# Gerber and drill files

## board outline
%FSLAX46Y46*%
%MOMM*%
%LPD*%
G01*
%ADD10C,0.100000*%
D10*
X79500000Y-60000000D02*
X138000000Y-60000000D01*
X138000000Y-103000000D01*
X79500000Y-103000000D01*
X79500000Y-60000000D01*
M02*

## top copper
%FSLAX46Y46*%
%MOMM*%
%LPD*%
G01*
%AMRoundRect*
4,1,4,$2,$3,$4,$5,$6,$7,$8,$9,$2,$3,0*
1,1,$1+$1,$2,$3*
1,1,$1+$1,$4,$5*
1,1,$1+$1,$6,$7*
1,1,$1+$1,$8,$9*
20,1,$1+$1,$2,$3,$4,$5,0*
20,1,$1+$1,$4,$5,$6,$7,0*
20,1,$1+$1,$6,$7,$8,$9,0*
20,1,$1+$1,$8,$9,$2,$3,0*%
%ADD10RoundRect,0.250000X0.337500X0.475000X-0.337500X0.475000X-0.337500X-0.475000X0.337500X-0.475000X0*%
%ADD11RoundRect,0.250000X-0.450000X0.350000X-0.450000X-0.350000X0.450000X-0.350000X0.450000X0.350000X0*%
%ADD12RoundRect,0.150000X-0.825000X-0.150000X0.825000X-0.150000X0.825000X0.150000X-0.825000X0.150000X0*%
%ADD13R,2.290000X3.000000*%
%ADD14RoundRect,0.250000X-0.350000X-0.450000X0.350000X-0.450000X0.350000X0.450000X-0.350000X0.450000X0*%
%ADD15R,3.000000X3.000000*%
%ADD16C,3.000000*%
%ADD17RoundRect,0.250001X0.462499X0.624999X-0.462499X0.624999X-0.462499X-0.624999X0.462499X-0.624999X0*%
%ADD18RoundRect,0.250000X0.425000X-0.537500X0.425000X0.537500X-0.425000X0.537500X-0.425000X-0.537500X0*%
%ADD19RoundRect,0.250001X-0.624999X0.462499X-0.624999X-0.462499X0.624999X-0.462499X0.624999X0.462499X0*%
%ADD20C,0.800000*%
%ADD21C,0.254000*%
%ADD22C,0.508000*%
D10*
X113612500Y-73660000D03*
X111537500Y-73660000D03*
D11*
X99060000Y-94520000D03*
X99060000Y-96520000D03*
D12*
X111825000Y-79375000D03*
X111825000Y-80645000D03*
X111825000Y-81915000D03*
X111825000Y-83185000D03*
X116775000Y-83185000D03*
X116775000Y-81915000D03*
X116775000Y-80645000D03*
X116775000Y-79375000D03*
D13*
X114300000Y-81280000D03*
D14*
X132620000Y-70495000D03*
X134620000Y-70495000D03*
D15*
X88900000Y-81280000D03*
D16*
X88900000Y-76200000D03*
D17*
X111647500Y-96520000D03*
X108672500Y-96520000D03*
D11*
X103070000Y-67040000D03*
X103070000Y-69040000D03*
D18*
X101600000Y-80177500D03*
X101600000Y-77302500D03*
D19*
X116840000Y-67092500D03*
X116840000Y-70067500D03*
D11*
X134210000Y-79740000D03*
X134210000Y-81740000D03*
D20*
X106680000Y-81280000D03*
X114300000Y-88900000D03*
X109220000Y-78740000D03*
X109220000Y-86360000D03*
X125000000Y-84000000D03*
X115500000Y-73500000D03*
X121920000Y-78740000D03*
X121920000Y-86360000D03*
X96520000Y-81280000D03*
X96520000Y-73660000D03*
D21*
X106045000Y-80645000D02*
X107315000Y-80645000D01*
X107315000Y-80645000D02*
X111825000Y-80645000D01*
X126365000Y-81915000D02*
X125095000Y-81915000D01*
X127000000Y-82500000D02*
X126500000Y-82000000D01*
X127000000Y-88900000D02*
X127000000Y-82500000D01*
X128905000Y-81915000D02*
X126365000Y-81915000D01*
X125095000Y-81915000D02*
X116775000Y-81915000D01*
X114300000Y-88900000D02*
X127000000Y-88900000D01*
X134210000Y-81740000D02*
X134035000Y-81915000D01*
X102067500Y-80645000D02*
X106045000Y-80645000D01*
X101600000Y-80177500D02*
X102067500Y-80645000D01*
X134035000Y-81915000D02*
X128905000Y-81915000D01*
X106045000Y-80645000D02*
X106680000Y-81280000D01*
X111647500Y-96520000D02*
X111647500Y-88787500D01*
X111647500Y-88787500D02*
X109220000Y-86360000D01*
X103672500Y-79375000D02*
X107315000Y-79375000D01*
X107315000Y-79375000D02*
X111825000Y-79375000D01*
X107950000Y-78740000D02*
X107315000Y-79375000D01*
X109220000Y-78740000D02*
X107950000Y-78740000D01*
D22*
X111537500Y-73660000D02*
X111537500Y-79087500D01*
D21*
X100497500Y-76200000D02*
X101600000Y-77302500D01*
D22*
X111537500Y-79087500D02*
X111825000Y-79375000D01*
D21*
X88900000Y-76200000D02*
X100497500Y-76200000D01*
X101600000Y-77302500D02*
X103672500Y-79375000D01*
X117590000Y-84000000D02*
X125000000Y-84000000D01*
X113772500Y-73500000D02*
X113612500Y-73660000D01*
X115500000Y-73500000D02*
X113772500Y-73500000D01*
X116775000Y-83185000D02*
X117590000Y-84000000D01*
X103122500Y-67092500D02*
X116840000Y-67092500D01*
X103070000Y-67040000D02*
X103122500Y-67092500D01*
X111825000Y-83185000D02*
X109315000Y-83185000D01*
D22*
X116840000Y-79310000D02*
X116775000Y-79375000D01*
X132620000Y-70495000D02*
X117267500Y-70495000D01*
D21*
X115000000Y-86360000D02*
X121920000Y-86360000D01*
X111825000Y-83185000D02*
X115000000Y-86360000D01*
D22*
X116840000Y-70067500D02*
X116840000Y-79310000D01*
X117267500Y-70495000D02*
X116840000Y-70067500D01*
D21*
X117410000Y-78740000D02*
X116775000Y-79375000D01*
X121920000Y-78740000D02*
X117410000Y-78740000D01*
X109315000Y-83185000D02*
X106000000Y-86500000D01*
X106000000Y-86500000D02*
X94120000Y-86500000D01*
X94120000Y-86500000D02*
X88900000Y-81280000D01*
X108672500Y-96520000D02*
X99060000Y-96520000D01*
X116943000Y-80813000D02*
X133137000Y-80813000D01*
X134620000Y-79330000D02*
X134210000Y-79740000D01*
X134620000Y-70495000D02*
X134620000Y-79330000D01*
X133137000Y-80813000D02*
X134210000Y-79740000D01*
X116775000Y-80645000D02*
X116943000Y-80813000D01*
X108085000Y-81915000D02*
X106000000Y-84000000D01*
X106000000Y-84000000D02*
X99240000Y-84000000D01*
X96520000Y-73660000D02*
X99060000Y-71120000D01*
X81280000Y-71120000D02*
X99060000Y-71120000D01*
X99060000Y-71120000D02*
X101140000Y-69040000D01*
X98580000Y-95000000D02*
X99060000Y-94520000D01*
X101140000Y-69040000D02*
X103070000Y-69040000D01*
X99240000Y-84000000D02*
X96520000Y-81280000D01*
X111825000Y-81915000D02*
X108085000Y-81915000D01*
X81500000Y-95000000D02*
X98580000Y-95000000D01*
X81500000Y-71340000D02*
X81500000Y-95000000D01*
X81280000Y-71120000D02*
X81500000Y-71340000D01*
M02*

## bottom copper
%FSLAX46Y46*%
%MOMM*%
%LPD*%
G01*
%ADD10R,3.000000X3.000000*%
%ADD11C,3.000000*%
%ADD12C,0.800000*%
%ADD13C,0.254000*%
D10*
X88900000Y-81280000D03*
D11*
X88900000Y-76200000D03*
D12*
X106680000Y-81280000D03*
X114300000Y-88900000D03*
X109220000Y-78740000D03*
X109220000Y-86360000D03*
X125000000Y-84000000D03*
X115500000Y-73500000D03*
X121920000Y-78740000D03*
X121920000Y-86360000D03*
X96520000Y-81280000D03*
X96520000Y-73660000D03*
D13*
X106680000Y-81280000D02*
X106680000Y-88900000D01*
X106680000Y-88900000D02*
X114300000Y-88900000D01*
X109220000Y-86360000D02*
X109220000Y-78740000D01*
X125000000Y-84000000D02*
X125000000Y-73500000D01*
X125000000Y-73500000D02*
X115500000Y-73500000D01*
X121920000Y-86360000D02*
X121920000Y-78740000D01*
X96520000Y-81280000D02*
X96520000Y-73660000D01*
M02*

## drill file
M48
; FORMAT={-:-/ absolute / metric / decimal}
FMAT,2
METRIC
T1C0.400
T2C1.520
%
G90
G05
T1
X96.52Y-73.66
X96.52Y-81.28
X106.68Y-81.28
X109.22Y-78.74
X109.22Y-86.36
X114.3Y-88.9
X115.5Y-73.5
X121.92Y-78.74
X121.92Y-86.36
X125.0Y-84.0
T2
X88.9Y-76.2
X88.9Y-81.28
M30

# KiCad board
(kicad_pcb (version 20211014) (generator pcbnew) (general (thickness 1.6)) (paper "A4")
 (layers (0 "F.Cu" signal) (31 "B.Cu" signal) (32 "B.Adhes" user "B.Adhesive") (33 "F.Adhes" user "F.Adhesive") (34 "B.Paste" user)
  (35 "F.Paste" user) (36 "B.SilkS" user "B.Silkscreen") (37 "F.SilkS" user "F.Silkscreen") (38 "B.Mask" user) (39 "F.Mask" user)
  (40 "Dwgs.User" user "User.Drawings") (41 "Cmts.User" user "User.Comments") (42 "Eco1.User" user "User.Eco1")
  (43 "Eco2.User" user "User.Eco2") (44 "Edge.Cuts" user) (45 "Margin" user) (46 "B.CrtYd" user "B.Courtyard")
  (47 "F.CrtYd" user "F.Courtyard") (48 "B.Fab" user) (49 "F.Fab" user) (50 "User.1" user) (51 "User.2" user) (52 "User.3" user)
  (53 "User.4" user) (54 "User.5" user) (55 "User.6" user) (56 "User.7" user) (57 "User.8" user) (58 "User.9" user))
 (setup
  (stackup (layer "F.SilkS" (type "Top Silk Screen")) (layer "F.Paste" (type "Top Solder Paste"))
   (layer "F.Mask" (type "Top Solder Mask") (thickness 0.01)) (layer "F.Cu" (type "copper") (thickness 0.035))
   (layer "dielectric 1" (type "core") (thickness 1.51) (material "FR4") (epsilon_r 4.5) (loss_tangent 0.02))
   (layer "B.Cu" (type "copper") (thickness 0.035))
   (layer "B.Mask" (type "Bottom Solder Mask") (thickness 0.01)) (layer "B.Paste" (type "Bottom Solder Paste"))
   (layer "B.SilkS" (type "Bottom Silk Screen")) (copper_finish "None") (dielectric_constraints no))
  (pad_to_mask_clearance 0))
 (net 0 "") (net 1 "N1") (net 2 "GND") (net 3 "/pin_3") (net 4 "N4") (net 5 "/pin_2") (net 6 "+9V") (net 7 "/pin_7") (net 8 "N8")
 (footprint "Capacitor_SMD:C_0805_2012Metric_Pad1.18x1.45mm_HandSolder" (layer "F.Cu") (at 112.575 73.66 180)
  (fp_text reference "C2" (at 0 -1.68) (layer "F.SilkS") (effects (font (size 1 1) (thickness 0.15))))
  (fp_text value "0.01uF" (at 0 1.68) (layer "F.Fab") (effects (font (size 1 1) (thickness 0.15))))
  (pad "1" smd roundrect (at -1.0375 0 180) (size 1.175 1.45) (layers "F.Cu" "F.Paste" "F.Mask") (roundrect_rratio 0.2127659574)
   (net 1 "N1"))
  (pad "2" smd roundrect (at 1.0375 0 180) (size 1.175 1.45) (layers "F.Cu" "F.Paste" "F.Mask") (roundrect_rratio 0.2127659574)
   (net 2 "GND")))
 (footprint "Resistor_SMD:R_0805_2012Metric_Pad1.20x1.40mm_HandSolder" (layer "F.Cu") (at 99.06 95.52 -90)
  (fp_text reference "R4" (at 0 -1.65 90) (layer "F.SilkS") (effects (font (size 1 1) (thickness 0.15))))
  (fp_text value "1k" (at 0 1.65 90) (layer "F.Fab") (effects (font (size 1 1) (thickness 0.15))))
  (pad "1" smd roundrect (at -1 0 270) (size 1.2 1.4) (layers "F.Cu" "F.Paste" "F.Mask") (roundrect_rratio 0.2083333333) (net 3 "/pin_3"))
  (pad "2" smd roundrect (at 1 0 270) (size 1.2 1.4) (layers "F.Cu" "F.Paste" "F.Mask") (roundrect_rratio 0.2083333333) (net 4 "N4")))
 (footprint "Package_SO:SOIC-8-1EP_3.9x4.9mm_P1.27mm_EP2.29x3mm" (layer "F.Cu") (at 114.3 81.28)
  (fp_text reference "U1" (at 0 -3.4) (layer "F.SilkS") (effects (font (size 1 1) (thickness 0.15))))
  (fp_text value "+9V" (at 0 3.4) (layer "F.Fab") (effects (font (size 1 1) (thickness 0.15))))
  (pad "" smd roundrect (at 0.57 0.75) (size 0.92 1.21) (layers "F.Paste") (roundrect_rratio 0.25))
  (pad "" smd roundrect (at 0.57 -0.75) (size 0.92 1.21) (layers "F.Paste") (roundrect_rratio 0.25))
  (pad "" smd roundrect (at -0.57 -0.75) (size 0.92 1.21) (layers "F.Paste") (roundrect_rratio 0.25))
  (pad "" smd roundrect (at -0.57 0.75) (size 0.92 1.21) (layers "F.Paste") (roundrect_rratio 0.25))
  (pad "1" smd roundrect (at -2.475 -1.905) (size 1.95 0.6) (layers "F.Cu" "F.Paste" "F.Mask") (roundrect_rratio 0.25) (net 2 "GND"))
  (pad "2" smd roundrect (at -2.475 -0.635) (size 1.95 0.6) (layers "F.Cu" "F.Paste" "F.Mask") (roundrect_rratio 0.25) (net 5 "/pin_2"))
  (pad "3" smd roundrect (at -2.475 0.635) (size 1.95 0.6) (layers "F.Cu" "F.Paste" "F.Mask") (roundrect_rratio 0.25) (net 3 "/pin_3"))
  (pad "4" smd roundrect (at -2.475 1.905) (size 1.95 0.6) (layers "F.Cu" "F.Paste" "F.Mask") (roundrect_rratio 0.25) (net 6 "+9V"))
  (pad "5" smd roundrect (at 2.475 1.905) (size 1.95 0.6) (layers "F.Cu" "F.Paste" "F.Mask") (roundrect_rratio 0.25) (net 1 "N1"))
  (pad "6" smd roundrect (at 2.475 0.635) (size 1.95 0.6) (layers "F.Cu" "F.Paste" "F.Mask") (roundrect_rratio 0.25) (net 5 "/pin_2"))
  (pad "7" smd roundrect (at 2.475 -0.635) (size 1.95 0.6) (layers "F.Cu" "F.Paste" "F.Mask") (roundrect_rratio 0.25) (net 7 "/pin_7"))
  (pad "8" smd roundrect (at 2.475 -1.905) (size 1.95 0.6) (layers "F.Cu" "F.Paste" "F.Mask") (roundrect_rratio 0.25) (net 6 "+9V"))
  (pad "9" smd rect (at 0 0) (size 2.29 3) (layers "F.Cu" "F.Mask")))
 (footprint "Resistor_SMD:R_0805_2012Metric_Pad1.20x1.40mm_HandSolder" (layer "F.Cu") (at 133.62 70.495)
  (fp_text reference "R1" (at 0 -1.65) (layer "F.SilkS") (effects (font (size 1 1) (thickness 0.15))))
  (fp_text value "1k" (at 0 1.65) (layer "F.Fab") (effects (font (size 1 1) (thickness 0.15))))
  (pad "1" smd roundrect (at -1 0) (size 1.2 1.4) (layers "F.Cu" "F.Paste" "F.Mask") (roundrect_rratio 0.2083333333) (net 6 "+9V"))
  (pad "2" smd roundrect (at 1 0) (size 1.2 1.4) (layers "F.Cu" "F.Paste" "F.Mask") (roundrect_rratio 0.2083333333) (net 7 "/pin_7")))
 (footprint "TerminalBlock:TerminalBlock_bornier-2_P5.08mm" (layer "F.Cu") (at 88.9 81.28 90)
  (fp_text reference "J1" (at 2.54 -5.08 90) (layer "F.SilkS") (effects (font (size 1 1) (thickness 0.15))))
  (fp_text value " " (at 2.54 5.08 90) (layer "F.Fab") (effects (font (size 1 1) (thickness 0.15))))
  (pad "1" thru_hole rect (at 0 0 90) (size 3 3) (drill 1.52) (layers *.Cu *.Mask) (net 6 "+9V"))
  (pad "2" thru_hole circle (at 5.08 0 90) (size 3 3) (drill 1.52) (layers *.Cu *.Mask) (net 2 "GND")))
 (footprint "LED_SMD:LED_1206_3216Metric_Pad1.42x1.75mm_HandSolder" (layer "F.Cu") (at 110.16 96.52 180)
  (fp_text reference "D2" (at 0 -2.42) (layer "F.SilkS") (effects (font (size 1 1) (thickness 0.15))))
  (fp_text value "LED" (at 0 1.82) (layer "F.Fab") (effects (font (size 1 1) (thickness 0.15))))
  (pad "1" smd roundrect (at -1.4875 0 180) (size 1.425 1.75) (layers "F.Cu" "F.Paste" "F.Mask") (roundrect_rratio 0.1754392982)
   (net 2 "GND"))
  (pad "2" smd roundrect (at 1.4875 0 180) (size 1.425 1.75) (layers "F.Cu" "F.Paste" "F.Mask") (roundrect_rratio 0.1754392982) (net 4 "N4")))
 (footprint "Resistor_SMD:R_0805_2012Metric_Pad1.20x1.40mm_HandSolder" (layer "F.Cu") (at 103.07 68.04 -90)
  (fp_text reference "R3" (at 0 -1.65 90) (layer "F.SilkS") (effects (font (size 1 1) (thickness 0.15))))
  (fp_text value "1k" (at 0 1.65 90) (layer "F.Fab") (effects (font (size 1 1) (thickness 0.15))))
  (pad "1" smd roundrect (at -1 0 270) (size 1.2 1.4) (layers "F.Cu" "F.Paste" "F.Mask") (roundrect_rratio 0.2083333333) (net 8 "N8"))
  (pad "2" smd roundrect (at 1 0 270) (size 1.2 1.4) (layers "F.Cu" "F.Paste" "F.Mask") (roundrect_rratio 0.2083333333) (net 3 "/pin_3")))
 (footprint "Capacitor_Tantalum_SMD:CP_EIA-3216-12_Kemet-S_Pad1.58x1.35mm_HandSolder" (layer "F.Cu") (at 101.6 78.74 90)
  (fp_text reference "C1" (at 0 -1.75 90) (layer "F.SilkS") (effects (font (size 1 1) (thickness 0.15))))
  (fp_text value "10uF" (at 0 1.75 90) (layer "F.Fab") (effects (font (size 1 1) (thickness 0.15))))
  (pad "1" smd roundrect (at -1.4375 0 90) (size 1.575 1.35) (layers "F.Cu" "F.Paste" "F.Mask") (roundrect_rratio 0.1851851852)
   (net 5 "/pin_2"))
  (pad "2" smd roundrect (at 1.4375 0 90) (size 1.575 1.35) (layers "F.Cu" "F.Paste" "F.Mask") (roundrect_rratio 0.1851851852) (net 2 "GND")))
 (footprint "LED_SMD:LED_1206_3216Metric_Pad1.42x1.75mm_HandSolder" (layer "F.Cu") (at 116.84 68.58 -90)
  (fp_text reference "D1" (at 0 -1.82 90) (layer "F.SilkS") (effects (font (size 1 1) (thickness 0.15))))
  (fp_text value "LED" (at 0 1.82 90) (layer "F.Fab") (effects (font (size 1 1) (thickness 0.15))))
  (pad "1" smd roundrect (at -1.4875 0 270) (size 1.425 1.75) (layers "F.Cu" "F.Paste" "F.Mask") (roundrect_rratio 0.1754392982)
   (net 8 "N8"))
  (pad "2" smd roundrect (at 1.4875 0 270) (size 1.425 1.75) (layers "F.Cu" "F.Paste" "F.Mask") (roundrect_rratio 0.1754392982)
   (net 6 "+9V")))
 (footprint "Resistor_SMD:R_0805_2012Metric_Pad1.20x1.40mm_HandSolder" (layer "F.Cu") (at 134.21 80.74 -90)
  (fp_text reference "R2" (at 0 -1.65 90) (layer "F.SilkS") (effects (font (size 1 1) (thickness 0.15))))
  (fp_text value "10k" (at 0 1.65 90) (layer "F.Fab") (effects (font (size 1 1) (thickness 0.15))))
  (pad "1" smd roundrect (at -1 0 270) (size 1.2 1.4) (layers "F.Cu" "F.Paste" "F.Mask") (roundrect_rratio 0.2083333333) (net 7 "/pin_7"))
  (pad "2" smd roundrect (at 1 0 270) (size 1.2 1.4) (layers "F.Cu" "F.Paste" "F.Mask") (roundrect_rratio 0.2083333333) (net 5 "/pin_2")))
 (gr_rect (start 79.5 60) (end 138 103) (layer "Edge.Cuts") (width 0.1) (fill none))
 (segment (start 106.045 80.645) (end 107.315 80.645) (width 0.254) (layer "F.Cu") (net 5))
 (segment (start 107.315 80.645) (end 111.825 80.645) (width 0.254) (layer "F.Cu") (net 5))
 (segment (start 126.365 81.915) (end 125.095 81.915) (width 0.254) (layer "F.Cu") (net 5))
 (segment (start 127 82.5) (end 126.5 82) (width 0.254) (layer "F.Cu") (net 5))
 (segment (start 127 88.9) (end 127 82.5) (width 0.254) (layer "F.Cu") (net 5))
 (segment (start 128.905 81.915) (end 126.365 81.915) (width 0.254) (layer "F.Cu") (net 5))
 (segment (start 125.095 81.915) (end 116.775 81.915) (width 0.254) (layer "F.Cu") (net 5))
 (segment (start 114.3 88.9) (end 127 88.9) (width 0.254) (layer "F.Cu") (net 5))
 (segment (start 134.21 81.74) (end 134.035 81.915) (width 0.254) (layer "F.Cu") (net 5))
 (segment (start 102.0675 80.645) (end 106.045 80.645) (width 0.254) (layer "F.Cu") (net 5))
 (segment (start 101.6 80.1775) (end 102.0675 80.645) (width 0.254) (layer "F.Cu") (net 5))
 (segment (start 134.035 81.915) (end 128.905 81.915) (width 0.254) (layer "F.Cu") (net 5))
 (segment (start 106.045 80.645) (end 106.68 81.28) (width 0.254) (layer "F.Cu") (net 5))
 (via (at 106.68 81.28) (size 0.8) (drill 0.4) (layers "F.Cu" "B.Cu") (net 5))
 (via (at 114.3 88.9) (size 0.8) (drill 0.4) (layers "F.Cu" "B.Cu") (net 5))
 (segment (start 106.68 81.28) (end 106.68 88.9) (width 0.254) (layer "B.Cu") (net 5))
 (segment (start 106.68 88.9) (end 114.3 88.9) (width 0.254) (layer "B.Cu") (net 5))
 (segment (start 111.6475 96.52) (end 111.6475 88.7875) (width 0.254) (layer "F.Cu") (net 2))
 (segment (start 111.6475 88.7875) (end 109.22 86.36) (width 0.254) (layer "F.Cu") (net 2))
 (segment (start 103.6725 79.375) (end 107.315 79.375) (width 0.254) (layer "F.Cu") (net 2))
 (segment (start 107.315 79.375) (end 111.825 79.375) (width 0.254) (layer "F.Cu") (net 2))
 (segment (start 107.95 78.74) (end 107.315 79.375) (width 0.254) (layer "F.Cu") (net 2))
 (segment (start 109.22 78.74) (end 107.95 78.74) (width 0.254) (layer "F.Cu") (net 2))
 (segment (start 111.5375 73.66) (end 111.5375 79.0875) (width 0.508) (layer "F.Cu") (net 2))
 (segment (start 100.4975 76.2) (end 101.6 77.3025) (width 0.254) (layer "F.Cu") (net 2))
 (segment (start 111.5375 79.0875) (end 111.825 79.375) (width 0.508) (layer "F.Cu") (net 2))
 (segment (start 88.9 76.2) (end 100.4975 76.2) (width 0.254) (layer "F.Cu") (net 2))
 (segment (start 101.6 77.3025) (end 103.6725 79.375) (width 0.254) (layer "F.Cu") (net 2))
 (via (at 109.22 78.74) (size 0.8) (drill 0.4) (layers "F.Cu" "B.Cu") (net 2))
 (via (at 109.22 86.36) (size 0.8) (drill 0.4) (layers "F.Cu" "B.Cu") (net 2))
 (segment (start 109.22 86.36) (end 109.22 78.74) (width 0.254) (layer "B.Cu") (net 2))
 (segment (start 117.59 84) (end 125 84) (width 0.254) (layer "F.Cu") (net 1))
 (segment (start 113.7725 73.5) (end 113.6125 73.66) (width 0.254) (layer "F.Cu") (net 1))
 (segment (start 115.5 73.5) (end 113.7725 73.5) (width 0.254) (layer "F.Cu") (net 1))
 (segment (start 116.775 83.185) (end 117.59 84) (width 0.254) (layer "F.Cu") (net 1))
 (via (at 125 84) (size 0.8) (drill 0.4) (layers "F.Cu" "B.Cu") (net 1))
 (via (at 115.5 73.5) (size 0.8) (drill 0.4) (layers "F.Cu" "B.Cu") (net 1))
 (segment (start 125 84) (end 125 73.5) (width 0.254) (layer "B.Cu") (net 1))
 (segment (start 125 73.5) (end 115.5 73.5) (width 0.254) (layer "B.Cu") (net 1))
 (segment (start 103.1225 67.0925) (end 116.84 67.0925) (width 0.254) (layer "F.Cu") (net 8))
 (segment (start 103.07 67.04) (end 103.1225 67.0925) (width 0.254) (layer "F.Cu") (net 8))
 (segment (start 111.825 83.185) (end 109.315 83.185) (width 0.254) (layer "F.Cu") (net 6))
 (segment (start 116.84 79.31) (end 116.775 79.375) (width 0.508) (layer "F.Cu") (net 6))
 (segment (start 132.62 70.495) (end 117.2675 70.495) (width 0.508) (layer "F.Cu") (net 6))
 (segment (start 115 86.36) (end 121.92 86.36) (width 0.254) (layer "F.Cu") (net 6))
 (segment (start 111.825 83.185) (end 115 86.36) (width 0.254) (layer "F.Cu") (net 6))
 (segment (start 116.84 70.0675) (end 116.84 79.31) (width 0.508) (layer "F.Cu") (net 6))
 (segment (start 117.2675 70.495) (end 116.84 70.0675) (width 0.508) (layer "F.Cu") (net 6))
 (segment (start 117.41 78.74) (end 116.775 79.375) (width 0.254) (layer "F.Cu") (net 6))
 (segment (start 121.92 78.74) (end 117.41 78.74) (width 0.254) (layer "F.Cu") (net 6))
 (segment (start 109.315 83.185) (end 106 86.5) (width 0.254) (layer "F.Cu") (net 6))
 (segment (start 106 86.5) (end 94.12 86.5) (width 0.254) (layer "F.Cu") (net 6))
 (segment (start 94.12 86.5) (end 88.9 81.28) (width 0.254) (layer "F.Cu") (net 6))
 (via (at 121.92 78.74) (size 0.8) (drill 0.4) (layers "F.Cu" "B.Cu") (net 6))
 (via (at 121.92 86.36) (size 0.8) (drill 0.4) (layers "F.Cu" "B.Cu") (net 6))
 (segment (start 121.92 86.36) (end 121.92 78.74) (width 0.254) (layer "B.Cu") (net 6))
 (segment (start 108.6725 96.52) (end 99.06 96.52) (width 0.254) (layer "F.Cu") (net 4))
 (segment (start 116.943 80.813) (end 133.137 80.813) (width 0.254) (layer "F.Cu") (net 7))
 (segment (start 134.62 79.33) (end 134.21 79.74) (width 0.254) (layer "F.Cu") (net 7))
 (segment (start 134.62 70.495) (end 134.62 79.33) (width 0.254) (layer "F.Cu") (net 7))
 (segment (start 133.137 80.813) (end 134.21 79.74) (width 0.254) (layer "F.Cu") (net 7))
 (segment (start 116.775 80.645) (end 116.943 80.813) (width 0.254) (layer "F.Cu") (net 7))
 (segment (start 108.085 81.915) (end 106 84) (width 0.254) (layer "F.Cu") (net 3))
 (segment (start 106 84) (end 99.24 84) (width 0.254) (layer "F.Cu") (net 3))
 (segment (start 96.52 73.66) (end 99.06 71.12) (width 0.254) (layer "F.Cu") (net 3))
 (segment (start 81.28 71.12) (end 99.06 71.12) (width 0.254) (layer "F.Cu") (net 3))
 (segment (start 99.06 71.12) (end 101.14 69.04) (width 0.254) (layer "F.Cu") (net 3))
 (segment (start 98.58 95) (end 99.06 94.52) (width 0.254) (layer "F.Cu") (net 3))
 (segment (start 101.14 69.04) (end 103.07 69.04) (width 0.254) (layer "F.Cu") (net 3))
 (segment (start 99.24 84) (end 96.52 81.28) (width 0.254) (layer "F.Cu") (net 3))
 (segment (start 111.825 81.915) (end 108.085 81.915) (width 0.254) (layer "F.Cu") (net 3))
 (segment (start 81.5 95) (end 98.58 95) (width 0.254) (layer "F.Cu") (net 3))
 (segment (start 81.5 71.34) (end 81.5 95) (width 0.254) (layer "F.Cu") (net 3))
 (segment (start 81.28 71.12) (end 81.5 71.34) (width 0.254) (layer "F.Cu") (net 3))
 (via (at 96.52 81.28) (size 0.8) (drill 0.4) (layers "F.Cu" "B.Cu") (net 3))
 (via (at 96.52 73.66) (size 0.8) (drill 0.4) (layers "F.Cu" "B.Cu") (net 3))
 (segment (start 96.52 81.28) (end 96.52 73.66) (width 0.254) (layer "B.Cu") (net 3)))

